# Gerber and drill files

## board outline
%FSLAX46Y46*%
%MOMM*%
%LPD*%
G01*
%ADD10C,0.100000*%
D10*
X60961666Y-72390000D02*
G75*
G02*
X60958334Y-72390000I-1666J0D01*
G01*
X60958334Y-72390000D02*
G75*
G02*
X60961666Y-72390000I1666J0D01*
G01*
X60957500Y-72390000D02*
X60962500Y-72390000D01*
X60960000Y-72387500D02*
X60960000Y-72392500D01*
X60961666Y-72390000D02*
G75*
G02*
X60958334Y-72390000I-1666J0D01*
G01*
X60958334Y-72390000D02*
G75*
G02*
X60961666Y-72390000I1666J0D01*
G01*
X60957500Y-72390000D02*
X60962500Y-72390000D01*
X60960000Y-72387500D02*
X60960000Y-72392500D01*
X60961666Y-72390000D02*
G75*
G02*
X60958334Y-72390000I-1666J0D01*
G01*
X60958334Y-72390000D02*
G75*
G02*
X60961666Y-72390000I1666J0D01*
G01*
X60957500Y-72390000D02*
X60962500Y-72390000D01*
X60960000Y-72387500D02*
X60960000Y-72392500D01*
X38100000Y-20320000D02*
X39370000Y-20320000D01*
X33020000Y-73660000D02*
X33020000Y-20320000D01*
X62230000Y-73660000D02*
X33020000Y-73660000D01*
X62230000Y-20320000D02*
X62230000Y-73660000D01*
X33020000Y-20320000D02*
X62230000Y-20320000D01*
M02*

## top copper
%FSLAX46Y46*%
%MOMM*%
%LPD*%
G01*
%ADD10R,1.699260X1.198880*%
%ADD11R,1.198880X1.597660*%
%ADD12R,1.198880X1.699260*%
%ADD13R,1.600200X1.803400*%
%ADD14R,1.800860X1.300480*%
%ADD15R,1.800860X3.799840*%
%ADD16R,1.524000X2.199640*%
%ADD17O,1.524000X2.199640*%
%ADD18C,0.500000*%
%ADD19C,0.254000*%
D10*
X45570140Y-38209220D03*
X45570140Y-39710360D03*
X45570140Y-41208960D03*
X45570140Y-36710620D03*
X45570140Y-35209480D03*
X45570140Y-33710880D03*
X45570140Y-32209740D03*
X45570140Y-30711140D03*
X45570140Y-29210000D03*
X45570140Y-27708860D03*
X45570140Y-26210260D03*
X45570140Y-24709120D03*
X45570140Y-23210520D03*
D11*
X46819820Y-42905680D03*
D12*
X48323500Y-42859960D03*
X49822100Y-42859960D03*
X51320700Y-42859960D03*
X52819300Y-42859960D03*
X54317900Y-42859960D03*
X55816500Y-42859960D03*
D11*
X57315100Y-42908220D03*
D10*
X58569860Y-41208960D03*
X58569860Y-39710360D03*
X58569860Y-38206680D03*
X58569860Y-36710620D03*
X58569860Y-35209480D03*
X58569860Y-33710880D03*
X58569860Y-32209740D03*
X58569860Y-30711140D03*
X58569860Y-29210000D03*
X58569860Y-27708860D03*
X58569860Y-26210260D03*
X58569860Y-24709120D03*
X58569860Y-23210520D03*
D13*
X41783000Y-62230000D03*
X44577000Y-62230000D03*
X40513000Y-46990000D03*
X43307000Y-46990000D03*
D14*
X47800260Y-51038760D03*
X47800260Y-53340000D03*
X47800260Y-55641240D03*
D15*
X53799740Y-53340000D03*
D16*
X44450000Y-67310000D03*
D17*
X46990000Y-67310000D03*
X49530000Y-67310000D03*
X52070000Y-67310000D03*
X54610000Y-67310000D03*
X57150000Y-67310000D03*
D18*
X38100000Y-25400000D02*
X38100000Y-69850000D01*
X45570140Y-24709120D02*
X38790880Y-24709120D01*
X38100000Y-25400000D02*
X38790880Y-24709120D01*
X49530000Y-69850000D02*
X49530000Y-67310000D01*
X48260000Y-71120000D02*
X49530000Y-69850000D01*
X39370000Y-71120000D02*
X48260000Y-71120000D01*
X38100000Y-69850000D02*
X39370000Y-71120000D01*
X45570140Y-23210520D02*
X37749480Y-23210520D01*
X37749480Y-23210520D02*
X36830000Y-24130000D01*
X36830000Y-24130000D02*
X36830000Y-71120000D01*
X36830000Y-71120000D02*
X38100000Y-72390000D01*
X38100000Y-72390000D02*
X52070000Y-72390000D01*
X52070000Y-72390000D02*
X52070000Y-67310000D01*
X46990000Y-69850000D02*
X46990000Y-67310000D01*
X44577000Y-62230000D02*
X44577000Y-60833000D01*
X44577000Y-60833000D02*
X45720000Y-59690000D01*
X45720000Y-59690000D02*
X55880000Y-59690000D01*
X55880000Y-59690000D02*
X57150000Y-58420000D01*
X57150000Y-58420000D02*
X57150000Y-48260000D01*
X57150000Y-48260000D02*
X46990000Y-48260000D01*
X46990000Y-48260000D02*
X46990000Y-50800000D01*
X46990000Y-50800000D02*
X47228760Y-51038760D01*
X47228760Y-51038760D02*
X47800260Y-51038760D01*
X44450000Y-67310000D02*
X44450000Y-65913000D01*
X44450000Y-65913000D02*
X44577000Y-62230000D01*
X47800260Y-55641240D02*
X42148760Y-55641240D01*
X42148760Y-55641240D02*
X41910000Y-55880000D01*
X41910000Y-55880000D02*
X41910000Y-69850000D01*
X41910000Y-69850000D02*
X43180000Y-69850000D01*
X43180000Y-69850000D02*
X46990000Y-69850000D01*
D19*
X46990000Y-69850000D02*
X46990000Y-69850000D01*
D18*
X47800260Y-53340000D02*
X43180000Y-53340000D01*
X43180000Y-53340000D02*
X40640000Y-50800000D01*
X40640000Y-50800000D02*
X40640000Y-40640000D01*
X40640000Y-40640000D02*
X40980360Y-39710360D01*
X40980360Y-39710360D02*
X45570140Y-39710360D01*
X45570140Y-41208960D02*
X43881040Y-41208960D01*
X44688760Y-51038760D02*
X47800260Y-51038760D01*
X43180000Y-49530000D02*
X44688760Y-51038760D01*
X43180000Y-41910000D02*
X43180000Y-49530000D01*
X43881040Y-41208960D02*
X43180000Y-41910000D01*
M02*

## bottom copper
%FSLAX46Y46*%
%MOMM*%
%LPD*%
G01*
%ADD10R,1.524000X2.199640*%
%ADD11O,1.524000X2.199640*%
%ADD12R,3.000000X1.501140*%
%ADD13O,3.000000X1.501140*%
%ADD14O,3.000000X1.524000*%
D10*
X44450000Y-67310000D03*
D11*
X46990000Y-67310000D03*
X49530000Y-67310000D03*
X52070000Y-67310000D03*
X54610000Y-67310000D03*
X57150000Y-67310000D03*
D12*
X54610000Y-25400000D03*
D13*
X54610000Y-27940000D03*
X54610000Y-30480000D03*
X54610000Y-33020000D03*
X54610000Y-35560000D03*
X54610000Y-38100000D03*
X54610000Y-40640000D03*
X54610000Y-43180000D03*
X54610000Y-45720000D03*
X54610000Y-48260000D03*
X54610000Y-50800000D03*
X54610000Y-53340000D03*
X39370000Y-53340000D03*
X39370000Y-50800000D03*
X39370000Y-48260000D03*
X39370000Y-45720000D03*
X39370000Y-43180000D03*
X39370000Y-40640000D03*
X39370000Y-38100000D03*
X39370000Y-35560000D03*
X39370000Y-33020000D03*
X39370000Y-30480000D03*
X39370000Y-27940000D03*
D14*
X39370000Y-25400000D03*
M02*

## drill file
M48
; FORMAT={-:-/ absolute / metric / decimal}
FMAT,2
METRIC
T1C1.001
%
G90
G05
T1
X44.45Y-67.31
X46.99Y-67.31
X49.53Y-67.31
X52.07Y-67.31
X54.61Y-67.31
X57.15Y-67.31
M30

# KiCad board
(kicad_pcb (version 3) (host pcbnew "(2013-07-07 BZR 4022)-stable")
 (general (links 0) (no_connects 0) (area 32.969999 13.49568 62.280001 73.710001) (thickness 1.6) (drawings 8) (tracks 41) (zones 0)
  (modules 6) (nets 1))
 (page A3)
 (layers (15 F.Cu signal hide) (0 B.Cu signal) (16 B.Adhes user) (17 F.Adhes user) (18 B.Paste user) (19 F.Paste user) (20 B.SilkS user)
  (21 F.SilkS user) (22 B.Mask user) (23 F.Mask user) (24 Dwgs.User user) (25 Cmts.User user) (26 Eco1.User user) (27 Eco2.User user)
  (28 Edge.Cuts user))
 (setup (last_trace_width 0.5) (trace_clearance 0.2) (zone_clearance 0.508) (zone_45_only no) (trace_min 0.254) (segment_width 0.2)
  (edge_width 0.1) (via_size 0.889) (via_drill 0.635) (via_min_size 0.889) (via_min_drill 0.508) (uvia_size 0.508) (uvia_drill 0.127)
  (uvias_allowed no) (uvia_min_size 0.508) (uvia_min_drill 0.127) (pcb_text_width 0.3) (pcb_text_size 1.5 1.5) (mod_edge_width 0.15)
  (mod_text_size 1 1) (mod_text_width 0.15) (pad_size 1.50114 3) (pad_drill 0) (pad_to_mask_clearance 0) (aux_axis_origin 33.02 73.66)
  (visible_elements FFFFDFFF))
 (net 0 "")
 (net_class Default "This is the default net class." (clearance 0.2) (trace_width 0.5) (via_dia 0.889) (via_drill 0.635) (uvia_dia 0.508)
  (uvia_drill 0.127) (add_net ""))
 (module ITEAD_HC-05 (layer F.Cu) (at 52.07 29.21)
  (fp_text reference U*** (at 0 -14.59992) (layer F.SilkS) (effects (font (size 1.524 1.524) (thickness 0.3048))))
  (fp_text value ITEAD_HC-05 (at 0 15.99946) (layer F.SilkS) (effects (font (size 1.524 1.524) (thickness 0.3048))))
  (pad 11 smd rect (at -6.49986 8.99922) (size 1.69926 1.19888) (layers F.Cu F.Paste F.Mask))
  (pad 12 smd rect (at -6.49986 10.50036) (size 1.69926 1.19888) (layers F.Cu F.Paste F.Mask))
  (pad 13 smd rect (at -6.49986 11.99896) (size 1.69926 1.19888) (layers F.Cu F.Paste F.Mask))
  (pad 10 smd rect (at -6.49986 7.50062) (size 1.69926 1.19888) (layers F.Cu F.Paste F.Mask))
  (pad 9 smd rect (at -6.49986 5.99948) (size 1.69926 1.19888) (layers F.Cu F.Paste F.Mask))
  (pad 8 smd rect (at -6.49986 4.50088) (size 1.69926 1.19888) (layers F.Cu F.Paste F.Mask))
  (pad 7 smd rect (at -6.49986 2.99974) (size 1.69926 1.19888) (layers F.Cu F.Paste F.Mask))
  (pad 6 smd rect (at -6.49986 1.50114) (size 1.69926 1.19888) (layers F.Cu F.Paste F.Mask))
  (pad 5 smd rect (at -6.49986 0) (size 1.69926 1.19888) (layers F.Cu F.Paste F.Mask))
  (pad 4 smd rect (at -6.49986 -1.50114) (size 1.69926 1.19888) (layers F.Cu F.Paste F.Mask))
  (pad 3 smd rect (at -6.49986 -2.99974) (size 1.69926 1.19888) (layers F.Cu F.Paste F.Mask))
  (pad 2 smd rect (at -6.49986 -4.50088) (size 1.69926 1.19888) (layers F.Cu F.Paste F.Mask))
  (pad 1 smd rect (at -6.49986 -5.99948) (size 1.69926 1.19888) (layers F.Cu F.Paste F.Mask))
  (pad 14 smd rect (at -5.25018 13.69568) (size 1.19888 1.59766) (layers F.Cu F.Paste F.Mask))
  (pad 15 smd rect (at -3.7465 13.64996) (size 1.19888 1.69926) (layers F.Cu F.Paste F.Mask))
  (pad 16 smd rect (at -2.2479 13.64996) (size 1.19888 1.69926) (layers F.Cu F.Paste F.Mask))
  (pad 17 smd rect (at -0.7493 13.64996) (size 1.19888 1.69926) (layers F.Cu F.Paste F.Mask))
  (pad 18 smd rect (at 0.7493 13.64996) (size 1.19888 1.69926) (layers F.Cu F.Paste F.Mask))
  (pad 19 smd rect (at 2.2479 13.64996) (size 1.19888 1.69926) (layers F.Cu F.Paste F.Mask))
  (pad 20 smd rect (at 3.7465 13.64996) (size 1.19888 1.69926) (layers F.Cu F.Paste F.Mask))
  (pad 21 smd rect (at 5.2451 13.69822) (size 1.19888 1.59766) (layers F.Cu F.Paste F.Mask))
  (pad 22 smd rect (at 6.49986 11.99896) (size 1.69926 1.19888) (layers F.Cu F.Paste F.Mask))
  (pad 23 smd rect (at 6.49986 10.50036) (size 1.69926 1.19888) (layers F.Cu F.Paste F.Mask))
  (pad 24 smd rect (at 6.49986 8.99668) (size 1.69926 1.19888) (layers F.Cu F.Paste F.Mask))
  (pad 25 smd rect (at 6.49986 7.50062) (size 1.69926 1.19888) (layers F.Cu F.Paste F.Mask))
  (pad 26 smd rect (at 6.49986 5.99948) (size 1.69926 1.19888) (layers F.Cu F.Paste F.Mask))
  (pad 27 smd rect (at 6.49986 4.50088) (size 1.69926 1.19888) (layers F.Cu F.Paste F.Mask))
  (pad 28 smd rect (at 6.49986 2.99974) (size 1.69926 1.19888) (layers F.Cu F.Paste F.Mask))
  (pad 29 smd rect (at 6.49986 1.50114) (size 1.69926 1.19888) (layers F.Cu F.Paste F.Mask))
  (pad 30 smd rect (at 6.49986 0) (size 1.69926 1.19888) (layers F.Cu F.Paste F.Mask))
  (pad 31 smd rect (at 6.49986 -1.50114) (size 1.69926 1.19888) (layers F.Cu F.Paste F.Mask))
  (pad 32 smd rect (at 6.49986 -2.99974) (size 1.69926 1.19888) (layers F.Cu F.Paste F.Mask))
  (pad 33 smd rect (at 6.49986 -4.50088) (size 1.69926 1.19888) (layers F.Cu F.Paste F.Mask))
  (pad 34 smd rect (at 6.49986 -5.99948) (size 1.69926 1.19888) (layers F.Cu F.Paste F.Mask)))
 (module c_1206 (layer F.Cu) (at 43.18 62.23 180)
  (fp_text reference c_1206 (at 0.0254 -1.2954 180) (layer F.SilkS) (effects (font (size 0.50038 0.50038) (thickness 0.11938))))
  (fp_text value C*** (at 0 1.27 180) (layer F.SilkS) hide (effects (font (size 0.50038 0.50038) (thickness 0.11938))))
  (pad 1 smd rect (at 1.397 0 180) (size 1.6002 1.8034) (layers F.Cu F.Paste F.Mask))
  (pad 2 smd rect (at -1.397 0 180) (size 1.6002 1.8034) (layers F.Cu F.Paste F.Mask)))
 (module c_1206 (layer F.Cu) (at 41.91 46.99 180)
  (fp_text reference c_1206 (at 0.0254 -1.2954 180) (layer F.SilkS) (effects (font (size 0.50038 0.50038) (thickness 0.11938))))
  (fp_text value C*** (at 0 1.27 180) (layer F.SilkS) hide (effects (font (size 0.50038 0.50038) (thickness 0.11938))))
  (pad 1 smd rect (at 1.397 0 180) (size 1.6002 1.8034) (layers F.Cu F.Paste F.Mask))
  (pad 2 smd rect (at -1.397 0 180) (size 1.6002 1.8034) (layers F.Cu F.Paste F.Mask)))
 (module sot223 (layer F.Cu) (at 50.8 53.34 270)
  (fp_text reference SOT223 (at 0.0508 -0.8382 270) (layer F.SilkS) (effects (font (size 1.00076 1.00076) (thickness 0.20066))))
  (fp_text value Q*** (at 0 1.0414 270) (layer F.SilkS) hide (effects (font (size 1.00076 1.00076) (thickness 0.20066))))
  (pad 1 smd rect (at -2.30124 2.99974 270) (size 1.30048 1.80086) (layers F.Cu F.Paste F.Mask))
  (pad 2 smd rect (at 0 2.99974 270) (size 1.30048 1.80086) (layers F.Cu F.Paste F.Mask))
  (pad 3 smd rect (at 2.30124 2.99974 270) (size 1.30048 1.80086) (layers F.Cu F.Paste F.Mask))
  (pad 4 smd rect (at 0 -2.99974 270) (size 3.79984 1.80086) (layers F.Cu F.Paste F.Mask)))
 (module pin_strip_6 (layer F.Cu) (at 50.8 67.31)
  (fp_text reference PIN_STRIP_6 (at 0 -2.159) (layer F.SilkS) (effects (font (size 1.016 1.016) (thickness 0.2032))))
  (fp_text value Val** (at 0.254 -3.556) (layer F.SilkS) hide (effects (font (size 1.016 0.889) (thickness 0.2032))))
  (pad 1 thru_hole rect (at -6.35 0) (size 1.524 2.19964) (drill 1.00076) (layers *.Cu *.Mask F.SilkS))
  (pad 2 thru_hole oval (at -3.81 0) (size 1.524 2.19964) (drill 1.00076) (layers *.Cu *.Mask F.SilkS))
  (pad 3 thru_hole oval (at -1.27 0) (size 1.524 2.19964) (drill 1.00076) (layers *.Cu *.Mask F.SilkS))
  (pad 4 thru_hole oval (at 1.27 0) (size 1.524 2.19964) (drill 1.00076) (layers *.Cu *.Mask F.SilkS))
  (pad 5 thru_hole oval (at 3.81 0) (size 1.524 2.19964) (drill 1.00076) (layers *.Cu *.Mask F.SilkS))
  (pad 6 thru_hole oval (at 6.35 0) (size 1.524 2.19964) (drill 1.00076) (layers *.Cu *.Mask F.SilkS)))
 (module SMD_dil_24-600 (layer B.Cu) (at 46.99 39.37 270)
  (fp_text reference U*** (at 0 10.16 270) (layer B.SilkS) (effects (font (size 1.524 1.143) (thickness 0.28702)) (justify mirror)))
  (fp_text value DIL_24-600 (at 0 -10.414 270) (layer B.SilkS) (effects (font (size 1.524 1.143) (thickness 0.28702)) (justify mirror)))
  (pad 1 smd rect (at -13.97 -7.62 270) (size 1.50114 3) (layers B.Cu B.Paste B.Mask))
  (pad 2 smd oval (at -11.43 -7.62 270) (size 1.50114 3) (layers B.Cu B.Paste B.Mask))
  (pad 3 smd oval (at -8.89 -7.62 270) (size 1.50114 3) (layers B.Cu B.Paste B.Mask))
  (pad 4 smd oval (at -6.35 -7.62 270) (size 1.50114 3) (layers B.Cu B.Paste B.Mask))
  (pad 5 smd oval (at -3.81 -7.62 270) (size 1.50114 3) (layers B.Cu B.Paste B.Mask))
  (pad 6 smd oval (at -1.27 -7.62 270) (size 1.50114 3) (layers B.Cu B.Paste B.Mask))
  (pad 7 smd oval (at 1.27 -7.62 270) (size 1.50114 3) (layers B.Cu B.Paste B.Mask))
  (pad 8 smd oval (at 3.81 -7.62 270) (size 1.50114 3) (layers B.Cu B.Paste B.Mask))
  (pad 9 smd oval (at 6.35 -7.62 270) (size 1.50114 3) (layers B.Cu B.Paste B.Mask))
  (pad 10 smd oval (at 8.89 -7.62 270) (size 1.50114 3) (layers B.Cu B.Paste B.Mask))
  (pad 11 smd oval (at 11.43 -7.62 270) (size 1.50114 3) (layers B.Cu B.Paste B.Mask))
  (pad 12 smd oval (at 13.97 -7.62 270) (size 1.50114 3) (layers B.Cu B.Paste B.Mask))
  (pad 13 smd oval (at 13.97 7.62 270) (size 1.50114 3) (layers B.Cu B.Paste B.Mask))
  (pad 14 smd oval (at 11.43 7.62 270) (size 1.50114 3) (layers B.Cu B.Paste B.Mask))
  (pad 15 smd oval (at 8.89 7.62 270) (size 1.50114 3) (layers B.Cu B.Paste B.Mask))
  (pad 16 smd oval (at 6.35 7.62 270) (size 1.50114 3) (layers B.Cu B.Paste B.Mask))
  (pad 17 smd oval (at 3.81 7.62 270) (size 1.50114 3) (layers B.Cu B.Paste B.Mask))
  (pad 18 smd oval (at 1.27 7.62 270) (size 1.50114 3) (layers B.Cu B.Paste B.Mask))
  (pad 19 smd oval (at -1.27 7.62 270) (size 1.50114 3) (layers B.Cu B.Paste B.Mask))
  (pad 20 smd oval (at -3.81 7.62 270) (size 1.50114 3) (layers B.Cu B.Paste B.Mask))
  (pad 21 smd oval (at -6.35 7.62 270) (size 1.50114 3) (layers B.Cu B.Paste B.Mask))
  (pad 22 smd oval (at -8.89 7.62 270) (size 1.50114 3) (layers B.Cu B.Paste B.Mask))
  (pad 23 smd oval (at -11.43 7.62 270) (size 1.50114 3) (layers B.Cu B.Paste B.Mask))
  (pad 24 smd oval (at -13.97 7.62 270) (size 1.524 3) (layers B.Cu B.Paste B.Mask)))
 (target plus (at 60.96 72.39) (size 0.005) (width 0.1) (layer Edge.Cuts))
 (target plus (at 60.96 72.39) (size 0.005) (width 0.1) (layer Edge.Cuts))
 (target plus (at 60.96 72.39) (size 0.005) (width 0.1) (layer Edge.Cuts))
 (gr_line (start 38.1 20.32) (end 39.37 20.32) (angle 90) (layer Edge.Cuts) (width 0.1))
 (gr_line (start 33.02 73.66) (end 33.02 20.32) (angle 90) (layer Edge.Cuts) (width 0.1))
 (gr_line (start 62.23 73.66) (end 33.02 73.66) (angle 90) (layer Edge.Cuts) (width 0.1))
 (gr_line (start 62.23 20.32) (end 62.23 73.66) (angle 90) (layer Edge.Cuts) (width 0.1))
 (gr_line (start 33.02 20.32) (end 62.23 20.32) (angle 90) (layer Edge.Cuts) (width 0.1))
 (segment (start 38.1 25.4) (end 38.1 69.85) (width 0.5) (layer F.Cu) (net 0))
 (segment (start 45.57014 24.70912) (end 38.79088 24.70912) (width 0.5) (layer F.Cu) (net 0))
 (segment (start 38.1 25.4) (end 38.79088 24.70912) (width 0.5) (layer F.Cu) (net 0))
 (segment (start 49.53 69.85) (end 49.53 67.31) (width 0.5) (layer F.Cu) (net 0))
 (segment (start 48.26 71.12) (end 49.53 69.85) (width 0.5) (layer F.Cu) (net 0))
 (segment (start 39.37 71.12) (end 48.26 71.12) (width 0.5) (layer F.Cu) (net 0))
 (segment (start 38.1 69.85) (end 39.37 71.12) (width 0.5) (layer F.Cu) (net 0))
 (segment (start 45.57014 23.21052) (end 37.74948 23.21052) (width 0.5) (layer F.Cu) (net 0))
 (segment (start 37.74948 23.21052) (end 36.83 24.13) (width 0.5) (layer F.Cu) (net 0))
 (segment (start 36.83 24.13) (end 36.83 71.12) (width 0.5) (layer F.Cu) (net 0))
 (segment (start 36.83 71.12) (end 38.1 72.39) (width 0.5) (layer F.Cu) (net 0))
 (segment (start 38.1 72.39) (end 52.07 72.39) (width 0.5) (layer F.Cu) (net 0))
 (segment (start 52.07 72.39) (end 52.07 67.31) (width 0.5) (layer F.Cu) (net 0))
 (segment (start 46.99 69.85) (end 46.99 67.31) (width 0.5) (layer F.Cu) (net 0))
 (segment (start 44.577 62.23) (end 44.577 60.833) (width 0.5) (layer F.Cu) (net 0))
 (segment (start 44.577 60.833) (end 45.72 59.69) (width 0.5) (layer F.Cu) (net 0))
 (segment (start 45.72 59.69) (end 55.88 59.69) (width 0.5) (layer F.Cu) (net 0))
 (segment (start 55.88 59.69) (end 57.15 58.42) (width 0.5) (layer F.Cu) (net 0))
 (segment (start 57.15 58.42) (end 57.15 48.26) (width 0.5) (layer F.Cu) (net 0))
 (segment (start 57.15 48.26) (end 46.99 48.26) (width 0.5) (layer F.Cu) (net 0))
 (segment (start 46.99 48.26) (end 46.99 50.8) (width 0.5) (layer F.Cu) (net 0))
 (segment (start 46.99 50.8) (end 47.22876 51.03876) (width 0.5) (layer F.Cu) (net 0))
 (segment (start 47.22876 51.03876) (end 47.80026 51.03876) (width 0.5) (layer F.Cu) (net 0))
 (segment (start 44.45 67.31) (end 44.45 65.913) (width 0.5) (layer F.Cu) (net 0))
 (segment (start 44.45 65.913) (end 44.577 62.23) (width 0.5) (layer F.Cu) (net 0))
 (segment (start 47.80026 55.64124) (end 42.14876 55.64124) (width 0.5) (layer F.Cu) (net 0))
 (segment (start 42.14876 55.64124) (end 41.91 55.88) (width 0.5) (layer F.Cu) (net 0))
 (segment (start 41.91 55.88) (end 41.91 69.85) (width 0.5) (layer F.Cu) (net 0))
 (segment (start 41.91 69.85) (end 43.18 69.85) (width 0.5) (layer F.Cu) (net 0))
 (segment (start 43.18 69.85) (end 46.99 69.85) (width 0.5) (layer F.Cu) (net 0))
 (segment (start 46.99 69.85) (end 46.99 69.85) (width 0.254) (layer F.Cu) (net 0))
 (segment (start 47.80026 53.34) (end 43.18 53.34) (width 0.5) (layer F.Cu) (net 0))
 (segment (start 43.18 53.34) (end 40.64 50.8) (width 0.5) (layer F.Cu) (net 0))
 (segment (start 40.64 50.8) (end 40.64 40.64) (width 0.5) (layer F.Cu) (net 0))
 (segment (start 40.64 40.64) (end 40.98036 39.71036) (width 0.5) (layer F.Cu) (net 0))
 (segment (start 40.98036 39.71036) (end 45.57014 39.71036) (width 0.5) (layer F.Cu) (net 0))
 (segment (start 45.57014 41.20896) (end 43.88104 41.20896) (width 0.5) (layer F.Cu) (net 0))
 (segment (start 44.68876 51.03876) (end 47.80026 51.03876) (width 0.5) (layer F.Cu) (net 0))
 (segment (start 43.18 49.53) (end 44.68876 51.03876) (width 0.5) (layer F.Cu) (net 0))
 (segment (start 43.18 41.91) (end 43.18 49.53) (width 0.5) (layer F.Cu) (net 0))
 (segment (start 43.88104 41.20896) (end 43.18 41.91) (width 0.5) (layer F.Cu) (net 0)))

